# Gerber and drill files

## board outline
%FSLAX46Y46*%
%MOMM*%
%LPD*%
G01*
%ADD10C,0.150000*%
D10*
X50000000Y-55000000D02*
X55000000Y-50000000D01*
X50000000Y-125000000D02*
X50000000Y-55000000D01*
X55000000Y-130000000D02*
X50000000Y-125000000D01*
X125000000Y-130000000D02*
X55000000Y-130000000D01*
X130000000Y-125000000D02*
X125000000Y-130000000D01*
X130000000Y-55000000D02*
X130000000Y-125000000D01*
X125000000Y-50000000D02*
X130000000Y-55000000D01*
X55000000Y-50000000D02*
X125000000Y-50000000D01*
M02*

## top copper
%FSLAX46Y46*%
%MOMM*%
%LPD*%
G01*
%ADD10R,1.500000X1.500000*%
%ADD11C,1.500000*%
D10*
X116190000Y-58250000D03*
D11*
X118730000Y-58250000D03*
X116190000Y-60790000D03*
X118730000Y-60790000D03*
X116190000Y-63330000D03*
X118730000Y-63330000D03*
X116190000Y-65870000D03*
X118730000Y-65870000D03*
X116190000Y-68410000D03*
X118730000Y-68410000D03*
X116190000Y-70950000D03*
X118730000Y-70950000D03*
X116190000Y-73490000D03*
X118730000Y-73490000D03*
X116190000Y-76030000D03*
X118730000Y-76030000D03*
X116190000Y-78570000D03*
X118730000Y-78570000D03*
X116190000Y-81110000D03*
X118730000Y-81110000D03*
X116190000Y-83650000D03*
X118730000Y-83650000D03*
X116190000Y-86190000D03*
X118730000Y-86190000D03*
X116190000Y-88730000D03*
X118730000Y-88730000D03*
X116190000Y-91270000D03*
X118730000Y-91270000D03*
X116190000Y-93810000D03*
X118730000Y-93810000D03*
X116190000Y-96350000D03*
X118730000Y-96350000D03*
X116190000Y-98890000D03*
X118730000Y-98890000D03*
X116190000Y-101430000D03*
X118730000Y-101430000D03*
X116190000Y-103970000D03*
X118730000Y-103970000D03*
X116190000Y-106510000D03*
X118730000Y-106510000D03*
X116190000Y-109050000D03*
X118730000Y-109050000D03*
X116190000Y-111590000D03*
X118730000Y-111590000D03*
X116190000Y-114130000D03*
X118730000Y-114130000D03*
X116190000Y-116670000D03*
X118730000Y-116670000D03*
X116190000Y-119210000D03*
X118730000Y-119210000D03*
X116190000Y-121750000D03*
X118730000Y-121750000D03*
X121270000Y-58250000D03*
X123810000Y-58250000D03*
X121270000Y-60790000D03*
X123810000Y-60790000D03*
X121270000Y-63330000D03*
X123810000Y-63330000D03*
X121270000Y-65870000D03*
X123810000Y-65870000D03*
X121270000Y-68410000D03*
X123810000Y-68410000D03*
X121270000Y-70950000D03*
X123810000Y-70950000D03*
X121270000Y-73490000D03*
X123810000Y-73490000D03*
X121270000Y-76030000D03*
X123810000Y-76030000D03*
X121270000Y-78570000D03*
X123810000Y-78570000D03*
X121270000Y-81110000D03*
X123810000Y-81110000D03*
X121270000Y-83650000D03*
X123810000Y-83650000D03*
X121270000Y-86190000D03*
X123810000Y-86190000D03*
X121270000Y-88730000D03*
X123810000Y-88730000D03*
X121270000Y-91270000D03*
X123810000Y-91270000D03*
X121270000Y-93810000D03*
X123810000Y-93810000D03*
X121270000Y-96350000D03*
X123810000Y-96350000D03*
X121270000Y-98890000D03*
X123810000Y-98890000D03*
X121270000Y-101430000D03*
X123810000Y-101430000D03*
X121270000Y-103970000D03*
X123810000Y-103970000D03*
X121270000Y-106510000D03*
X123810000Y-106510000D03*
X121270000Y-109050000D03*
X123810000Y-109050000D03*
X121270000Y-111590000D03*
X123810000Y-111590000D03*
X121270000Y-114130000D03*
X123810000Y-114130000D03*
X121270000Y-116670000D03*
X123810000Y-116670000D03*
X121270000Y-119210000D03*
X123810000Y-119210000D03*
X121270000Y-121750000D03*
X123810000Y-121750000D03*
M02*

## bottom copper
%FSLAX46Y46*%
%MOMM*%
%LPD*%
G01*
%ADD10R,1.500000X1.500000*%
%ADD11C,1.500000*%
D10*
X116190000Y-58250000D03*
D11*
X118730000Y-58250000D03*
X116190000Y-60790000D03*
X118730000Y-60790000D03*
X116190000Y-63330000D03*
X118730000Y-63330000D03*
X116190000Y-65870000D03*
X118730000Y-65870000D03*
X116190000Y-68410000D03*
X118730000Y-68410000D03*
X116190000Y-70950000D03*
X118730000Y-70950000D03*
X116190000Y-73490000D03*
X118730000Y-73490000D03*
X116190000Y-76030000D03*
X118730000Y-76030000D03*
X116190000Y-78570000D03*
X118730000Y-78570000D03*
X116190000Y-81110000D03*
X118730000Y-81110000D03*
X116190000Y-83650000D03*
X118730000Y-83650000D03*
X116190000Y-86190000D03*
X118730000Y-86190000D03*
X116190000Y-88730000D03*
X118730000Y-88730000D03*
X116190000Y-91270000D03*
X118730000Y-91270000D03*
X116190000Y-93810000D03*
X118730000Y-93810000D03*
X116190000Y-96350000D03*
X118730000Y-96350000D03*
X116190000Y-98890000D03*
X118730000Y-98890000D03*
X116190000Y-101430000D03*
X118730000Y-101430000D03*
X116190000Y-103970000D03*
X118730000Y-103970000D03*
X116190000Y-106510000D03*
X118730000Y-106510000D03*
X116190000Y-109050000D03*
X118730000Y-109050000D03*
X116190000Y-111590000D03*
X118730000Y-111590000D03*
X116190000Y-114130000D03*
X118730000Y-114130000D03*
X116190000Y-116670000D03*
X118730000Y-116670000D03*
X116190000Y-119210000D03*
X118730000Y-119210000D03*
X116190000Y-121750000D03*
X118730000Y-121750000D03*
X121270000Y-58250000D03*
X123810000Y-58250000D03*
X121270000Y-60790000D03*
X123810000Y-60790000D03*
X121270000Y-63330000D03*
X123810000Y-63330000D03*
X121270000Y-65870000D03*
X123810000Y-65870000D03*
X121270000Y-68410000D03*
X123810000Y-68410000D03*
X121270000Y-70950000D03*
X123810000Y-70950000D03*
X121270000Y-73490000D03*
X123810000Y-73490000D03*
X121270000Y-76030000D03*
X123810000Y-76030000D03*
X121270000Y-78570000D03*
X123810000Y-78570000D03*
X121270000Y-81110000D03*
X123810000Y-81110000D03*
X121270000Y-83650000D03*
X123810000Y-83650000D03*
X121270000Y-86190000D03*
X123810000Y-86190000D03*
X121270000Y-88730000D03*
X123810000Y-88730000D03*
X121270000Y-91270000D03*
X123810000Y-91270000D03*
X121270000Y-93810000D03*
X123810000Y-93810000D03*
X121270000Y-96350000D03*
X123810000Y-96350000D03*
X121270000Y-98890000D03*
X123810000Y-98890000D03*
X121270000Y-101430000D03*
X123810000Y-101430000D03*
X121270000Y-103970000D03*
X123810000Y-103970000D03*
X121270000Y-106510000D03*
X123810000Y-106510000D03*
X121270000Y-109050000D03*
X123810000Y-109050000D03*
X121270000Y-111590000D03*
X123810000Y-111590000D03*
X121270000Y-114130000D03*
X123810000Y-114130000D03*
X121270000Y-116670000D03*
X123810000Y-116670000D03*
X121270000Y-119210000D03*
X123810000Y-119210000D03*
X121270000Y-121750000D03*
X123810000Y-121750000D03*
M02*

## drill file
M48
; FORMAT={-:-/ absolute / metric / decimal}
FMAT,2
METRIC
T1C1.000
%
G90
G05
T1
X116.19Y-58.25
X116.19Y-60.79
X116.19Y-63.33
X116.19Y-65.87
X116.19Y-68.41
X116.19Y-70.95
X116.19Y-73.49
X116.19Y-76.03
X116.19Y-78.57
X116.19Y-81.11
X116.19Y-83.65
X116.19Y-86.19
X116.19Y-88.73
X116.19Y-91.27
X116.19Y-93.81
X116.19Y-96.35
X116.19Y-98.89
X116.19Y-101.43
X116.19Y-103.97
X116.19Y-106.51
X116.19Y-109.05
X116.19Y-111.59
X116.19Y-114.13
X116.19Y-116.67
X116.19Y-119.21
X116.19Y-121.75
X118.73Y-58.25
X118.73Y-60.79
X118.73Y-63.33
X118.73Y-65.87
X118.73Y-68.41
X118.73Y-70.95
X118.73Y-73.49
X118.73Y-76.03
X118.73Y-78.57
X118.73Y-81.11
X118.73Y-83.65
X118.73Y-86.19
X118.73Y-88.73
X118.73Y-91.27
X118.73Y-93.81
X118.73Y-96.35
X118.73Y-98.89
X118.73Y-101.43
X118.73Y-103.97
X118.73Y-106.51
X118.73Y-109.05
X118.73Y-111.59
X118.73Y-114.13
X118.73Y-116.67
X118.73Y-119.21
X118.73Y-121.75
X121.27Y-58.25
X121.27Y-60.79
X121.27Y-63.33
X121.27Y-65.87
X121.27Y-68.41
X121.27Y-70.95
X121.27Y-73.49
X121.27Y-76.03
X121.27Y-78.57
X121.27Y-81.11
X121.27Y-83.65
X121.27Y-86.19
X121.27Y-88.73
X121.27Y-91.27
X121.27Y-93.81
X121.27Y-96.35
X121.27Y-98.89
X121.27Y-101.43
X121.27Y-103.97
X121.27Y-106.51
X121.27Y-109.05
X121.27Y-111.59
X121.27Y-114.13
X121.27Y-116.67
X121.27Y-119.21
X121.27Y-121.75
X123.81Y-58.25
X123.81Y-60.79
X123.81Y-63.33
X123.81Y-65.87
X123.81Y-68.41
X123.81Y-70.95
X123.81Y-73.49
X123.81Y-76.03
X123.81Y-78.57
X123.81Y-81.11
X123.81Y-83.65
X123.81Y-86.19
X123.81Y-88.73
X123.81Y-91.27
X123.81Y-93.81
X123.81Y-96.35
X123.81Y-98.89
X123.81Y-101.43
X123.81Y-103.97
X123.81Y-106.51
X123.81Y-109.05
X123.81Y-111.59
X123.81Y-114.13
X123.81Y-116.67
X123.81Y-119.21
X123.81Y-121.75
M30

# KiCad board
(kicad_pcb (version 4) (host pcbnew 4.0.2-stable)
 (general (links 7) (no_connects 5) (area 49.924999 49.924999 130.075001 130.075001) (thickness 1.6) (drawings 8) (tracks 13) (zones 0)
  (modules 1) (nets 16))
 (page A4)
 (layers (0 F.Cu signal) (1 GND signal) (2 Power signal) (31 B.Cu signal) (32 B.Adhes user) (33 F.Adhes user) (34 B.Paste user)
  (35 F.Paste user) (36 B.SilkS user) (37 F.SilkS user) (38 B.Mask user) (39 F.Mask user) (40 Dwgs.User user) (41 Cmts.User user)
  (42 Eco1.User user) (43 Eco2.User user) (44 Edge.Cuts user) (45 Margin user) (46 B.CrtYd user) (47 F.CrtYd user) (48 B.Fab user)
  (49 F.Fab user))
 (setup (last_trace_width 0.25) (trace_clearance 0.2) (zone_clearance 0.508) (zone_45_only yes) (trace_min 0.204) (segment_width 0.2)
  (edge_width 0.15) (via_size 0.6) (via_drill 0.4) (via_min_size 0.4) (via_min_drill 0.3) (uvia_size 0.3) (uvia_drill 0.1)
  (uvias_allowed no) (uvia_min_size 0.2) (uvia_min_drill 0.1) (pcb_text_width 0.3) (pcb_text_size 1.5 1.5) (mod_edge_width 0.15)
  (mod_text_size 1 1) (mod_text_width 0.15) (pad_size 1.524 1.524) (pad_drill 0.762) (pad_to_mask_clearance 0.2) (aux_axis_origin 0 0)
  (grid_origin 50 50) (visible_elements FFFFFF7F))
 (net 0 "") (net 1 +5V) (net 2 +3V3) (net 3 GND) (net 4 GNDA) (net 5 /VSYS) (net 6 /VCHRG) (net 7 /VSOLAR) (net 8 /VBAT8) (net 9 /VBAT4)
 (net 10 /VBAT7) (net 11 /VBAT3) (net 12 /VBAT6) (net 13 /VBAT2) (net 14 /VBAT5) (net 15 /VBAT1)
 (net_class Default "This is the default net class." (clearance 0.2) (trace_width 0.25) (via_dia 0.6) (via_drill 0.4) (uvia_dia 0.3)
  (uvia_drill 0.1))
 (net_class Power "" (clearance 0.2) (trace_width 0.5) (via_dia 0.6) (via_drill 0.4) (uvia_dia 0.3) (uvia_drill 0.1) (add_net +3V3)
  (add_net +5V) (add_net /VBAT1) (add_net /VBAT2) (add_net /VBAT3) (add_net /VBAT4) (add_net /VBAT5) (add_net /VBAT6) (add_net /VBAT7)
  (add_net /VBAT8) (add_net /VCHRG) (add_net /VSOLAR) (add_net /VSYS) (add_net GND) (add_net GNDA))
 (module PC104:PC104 (layer F.Cu) (at 120 90)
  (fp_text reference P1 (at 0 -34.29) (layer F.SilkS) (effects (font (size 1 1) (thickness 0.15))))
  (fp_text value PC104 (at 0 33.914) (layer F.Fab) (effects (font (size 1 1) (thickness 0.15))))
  (pad 1A thru_hole rect (at -3.81 -31.75) (size 1.5 1.5) (drill 1) (layers *.Cu *.Mask F.SilkS))
  (pad 1B thru_hole circle (at -1.27 -31.75) (size 1.5 1.5) (drill 1) (layers *.Cu *.Mask F.SilkS))
  (pad 2A thru_hole circle (at -3.81 -29.21) (size 1.5 1.5) (drill 1) (layers *.Cu *.Mask F.SilkS))
  (pad 2B thru_hole circle (at -1.27 -29.21) (size 1.5 1.5) (drill 1) (layers *.Cu *.Mask F.SilkS))
  (pad 3A thru_hole circle (at -3.81 -26.67) (size 1.5 1.5) (drill 1) (layers *.Cu *.Mask F.SilkS))
  (pad 3B thru_hole circle (at -1.27 -26.67) (size 1.5 1.5) (drill 1) (layers *.Cu *.Mask F.SilkS))
  (pad 4A thru_hole circle (at -3.81 -24.13) (size 1.5 1.5) (drill 1) (layers *.Cu *.Mask F.SilkS))
  (pad 4B thru_hole circle (at -1.27 -24.13) (size 1.5 1.5) (drill 1) (layers *.Cu *.Mask F.SilkS))
  (pad 5A thru_hole circle (at -3.81 -21.59) (size 1.5 1.5) (drill 1) (layers *.Cu *.Mask F.SilkS))
  (pad 5B thru_hole circle (at -1.27 -21.59) (size 1.5 1.5) (drill 1) (layers *.Cu *.Mask F.SilkS))
  (pad 6A thru_hole circle (at -3.81 -19.05) (size 1.5 1.5) (drill 1) (layers *.Cu *.Mask F.SilkS))
  (pad 6B thru_hole circle (at -1.27 -19.05) (size 1.5 1.5) (drill 1) (layers *.Cu *.Mask F.SilkS))
  (pad 7A thru_hole circle (at -3.81 -16.51) (size 1.5 1.5) (drill 1) (layers *.Cu *.Mask F.SilkS))
  (pad 7B thru_hole circle (at -1.27 -16.51) (size 1.5 1.5) (drill 1) (layers *.Cu *.Mask F.SilkS))
  (pad 8A thru_hole circle (at -3.81 -13.97) (size 1.5 1.5) (drill 1) (layers *.Cu *.Mask F.SilkS))
  (pad 8B thru_hole circle (at -1.27 -13.97) (size 1.5 1.5) (drill 1) (layers *.Cu *.Mask F.SilkS))
  (pad 9A thru_hole circle (at -3.81 -11.43) (size 1.5 1.5) (drill 1) (layers *.Cu *.Mask F.SilkS))
  (pad 9B thru_hole circle (at -1.27 -11.43) (size 1.5 1.5) (drill 1) (layers *.Cu *.Mask F.SilkS))
  (pad 10A thru_hole circle (at -3.81 -8.89) (size 1.5 1.5) (drill 1) (layers *.Cu *.Mask F.SilkS))
  (pad 10B thru_hole circle (at -1.27 -8.89) (size 1.5 1.5) (drill 1) (layers *.Cu *.Mask F.SilkS))
  (pad 11A thru_hole circle (at -3.81 -6.35) (size 1.5 1.5) (drill 1) (layers *.Cu *.Mask F.SilkS))
  (pad 11B thru_hole circle (at -1.27 -6.35) (size 1.5 1.5) (drill 1) (layers *.Cu *.Mask F.SilkS))
  (pad 12A thru_hole circle (at -3.81 -3.81) (size 1.5 1.5) (drill 1) (layers *.Cu *.Mask F.SilkS))
  (pad 12B thru_hole circle (at -1.27 -3.81) (size 1.5 1.5) (drill 1) (layers *.Cu *.Mask F.SilkS))
  (pad 13A thru_hole circle (at -3.81 -1.27) (size 1.5 1.5) (drill 1) (layers *.Cu *.Mask F.SilkS))
  (pad 13B thru_hole circle (at -1.27 -1.27) (size 1.5 1.5) (drill 1) (layers *.Cu *.Mask F.SilkS))
  (pad 14A thru_hole circle (at -3.81 1.27) (size 1.5 1.5) (drill 1) (layers *.Cu *.Mask F.SilkS))
  (pad 14B thru_hole circle (at -1.27 1.27) (size 1.5 1.5) (drill 1) (layers *.Cu *.Mask F.SilkS))
  (pad 15A thru_hole circle (at -3.81 3.81) (size 1.5 1.5) (drill 1) (layers *.Cu *.Mask F.SilkS))
  (pad 15B thru_hole circle (at -1.27 3.81) (size 1.5 1.5) (drill 1) (layers *.Cu *.Mask F.SilkS))
  (pad 16A thru_hole circle (at -3.81 6.35) (size 1.5 1.5) (drill 1) (layers *.Cu *.Mask F.SilkS))
  (pad 16B thru_hole circle (at -1.27 6.35) (size 1.5 1.5) (drill 1) (layers *.Cu *.Mask F.SilkS))
  (pad 17A thru_hole circle (at -3.81 8.89) (size 1.5 1.5) (drill 1) (layers *.Cu *.Mask F.SilkS))
  (pad 17B thru_hole circle (at -1.27 8.89) (size 1.5 1.5) (drill 1) (layers *.Cu *.Mask F.SilkS))
  (pad 18A thru_hole circle (at -3.81 11.43) (size 1.5 1.5) (drill 1) (layers *.Cu *.Mask F.SilkS))
  (pad 18B thru_hole circle (at -1.27 11.43) (size 1.5 1.5) (drill 1) (layers *.Cu *.Mask F.SilkS))
  (pad 19A thru_hole circle (at -3.81 13.97) (size 1.5 1.5) (drill 1) (layers *.Cu *.Mask F.SilkS))
  (pad 19B thru_hole circle (at -1.27 13.97) (size 1.5 1.5) (drill 1) (layers *.Cu *.Mask F.SilkS))
  (pad 20A thru_hole circle (at -3.81 16.51) (size 1.5 1.5) (drill 1) (layers *.Cu *.Mask F.SilkS))
  (pad 20B thru_hole circle (at -1.27 16.51) (size 1.5 1.5) (drill 1) (layers *.Cu *.Mask F.SilkS))
  (pad 21A thru_hole circle (at -3.81 19.05) (size 1.5 1.5) (drill 1) (layers *.Cu *.Mask F.SilkS))
  (pad 21B thru_hole circle (at -1.27 19.05) (size 1.5 1.5) (drill 1) (layers *.Cu *.Mask F.SilkS))
  (pad 22A thru_hole circle (at -3.81 21.59) (size 1.5 1.5) (drill 1) (layers *.Cu *.Mask F.SilkS))
  (pad 22B thru_hole circle (at -1.27 21.59) (size 1.5 1.5) (drill 1) (layers *.Cu *.Mask F.SilkS))
  (pad 23A thru_hole circle (at -3.81 24.13) (size 1.5 1.5) (drill 1) (layers *.Cu *.Mask F.SilkS))
  (pad 23B thru_hole circle (at -1.27 24.13) (size 1.5 1.5) (drill 1) (layers *.Cu *.Mask F.SilkS))
  (pad 24A thru_hole circle (at -3.81 26.67) (size 1.5 1.5) (drill 1) (layers *.Cu *.Mask F.SilkS))
  (pad 24B thru_hole circle (at -1.27 26.67) (size 1.5 1.5) (drill 1) (layers *.Cu *.Mask F.SilkS))
  (pad 25A thru_hole circle (at -3.81 29.21) (size 1.5 1.5) (drill 1) (layers *.Cu *.Mask F.SilkS))
  (pad 25B thru_hole circle (at -1.27 29.21) (size 1.5 1.5) (drill 1) (layers *.Cu *.Mask F.SilkS))
  (pad 26A thru_hole circle (at -3.81 31.75) (size 1.5 1.5) (drill 1) (layers *.Cu *.Mask F.SilkS))
  (pad 26B thru_hole circle (at -1.27 31.75) (size 1.5 1.5) (drill 1) (layers *.Cu *.Mask F.SilkS))
  (pad 1C thru_hole circle (at 1.27 -31.75) (size 1.5 1.5) (drill 1) (layers *.Cu *.Mask F.SilkS))
  (pad 1D thru_hole circle (at 3.81 -31.75) (size 1.5 1.5) (drill 1) (layers *.Cu *.Mask F.SilkS))
  (pad 2C thru_hole circle (at 1.27 -29.21) (size 1.5 1.5) (drill 1) (layers *.Cu *.Mask F.SilkS))
  (pad 2D thru_hole circle (at 3.81 -29.21) (size 1.5 1.5) (drill 1) (layers *.Cu *.Mask F.SilkS))
  (pad 3C thru_hole circle (at 1.27 -26.67) (size 1.5 1.5) (drill 1) (layers *.Cu *.Mask F.SilkS))
  (pad 3D thru_hole circle (at 3.81 -26.67) (size 1.5 1.5) (drill 1) (layers *.Cu *.Mask F.SilkS))
  (pad 4C thru_hole circle (at 1.27 -24.13) (size 1.5 1.5) (drill 1) (layers *.Cu *.Mask F.SilkS))
  (pad 4D thru_hole circle (at 3.81 -24.13) (size 1.5 1.5) (drill 1) (layers *.Cu *.Mask F.SilkS))
  (pad 5C thru_hole circle (at 1.27 -21.59) (size 1.5 1.5) (drill 1) (layers *.Cu *.Mask F.SilkS))
  (pad 5D thru_hole circle (at 3.81 -21.59) (size 1.5 1.5) (drill 1) (layers *.Cu *.Mask F.SilkS))
  (pad 6C thru_hole circle (at 1.27 -19.05) (size 1.5 1.5) (drill 1) (layers *.Cu *.Mask F.SilkS))
  (pad 6D thru_hole circle (at 3.81 -19.05) (size 1.5 1.5) (drill 1) (layers *.Cu *.Mask F.SilkS))
  (pad 7C thru_hole circle (at 1.27 -16.51) (size 1.5 1.5) (drill 1) (layers *.Cu *.Mask F.SilkS))
  (pad 7D thru_hole circle (at 3.81 -16.51) (size 1.5 1.5) (drill 1) (layers *.Cu *.Mask F.SilkS))
  (pad 8C thru_hole circle (at 1.27 -13.97) (size 1.5 1.5) (drill 1) (layers *.Cu *.Mask F.SilkS))
  (pad 8D thru_hole circle (at 3.81 -13.97) (size 1.5 1.5) (drill 1) (layers *.Cu *.Mask F.SilkS))
  (pad 9C thru_hole circle (at 1.27 -11.43) (size 1.5 1.5) (drill 1) (layers *.Cu *.Mask F.SilkS))
  (pad 9D thru_hole circle (at 3.81 -11.43) (size 1.5 1.5) (drill 1) (layers *.Cu *.Mask F.SilkS))
  (pad 10C thru_hole circle (at 1.27 -8.89) (size 1.5 1.5) (drill 1) (layers *.Cu *.Mask F.SilkS))
  (pad 10D thru_hole circle (at 3.81 -8.89) (size 1.5 1.5) (drill 1) (layers *.Cu *.Mask F.SilkS))
  (pad 11C thru_hole circle (at 1.27 -6.35) (size 1.5 1.5) (drill 1) (layers *.Cu *.Mask F.SilkS))
  (pad 11D thru_hole circle (at 3.81 -6.35) (size 1.5 1.5) (drill 1) (layers *.Cu *.Mask F.SilkS))
  (pad 12C thru_hole circle (at 1.27 -3.81) (size 1.5 1.5) (drill 1) (layers *.Cu *.Mask F.SilkS))
  (pad 12D thru_hole circle (at 3.81 -3.81) (size 1.5 1.5) (drill 1) (layers *.Cu *.Mask F.SilkS))
  (pad 13C thru_hole circle (at 1.27 -1.27) (size 1.5 1.5) (drill 1) (layers *.Cu *.Mask F.SilkS) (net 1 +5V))
  (pad 13D thru_hole circle (at 3.81 -1.27) (size 1.5 1.5) (drill 1) (layers *.Cu *.Mask F.SilkS) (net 1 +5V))
  (pad 14C thru_hole circle (at 1.27 1.27) (size 1.5 1.5) (drill 1) (layers *.Cu *.Mask F.SilkS) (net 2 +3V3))
  (pad 14D thru_hole circle (at 3.81 1.27) (size 1.5 1.5) (drill 1) (layers *.Cu *.Mask F.SilkS) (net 2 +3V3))
  (pad 15C thru_hole circle (at 1.27 3.81) (size 1.5 1.5) (drill 1) (layers *.Cu *.Mask F.SilkS) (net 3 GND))
  (pad 15D thru_hole circle (at 3.81 3.81) (size 1.5 1.5) (drill 1) (layers *.Cu *.Mask F.SilkS) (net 3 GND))
  (pad 16C thru_hole circle (at 1.27 6.35) (size 1.5 1.5) (drill 1) (layers *.Cu *.Mask F.SilkS) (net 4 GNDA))
  (pad 16D thru_hole circle (at 3.81 6.35) (size 1.5 1.5) (drill 1) (layers *.Cu *.Mask F.SilkS) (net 3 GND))
  (pad 17C thru_hole circle (at 1.27 8.89) (size 1.5 1.5) (drill 1) (layers *.Cu *.Mask F.SilkS) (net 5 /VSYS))
  (pad 17D thru_hole circle (at 3.81 8.89) (size 1.5 1.5) (drill 1) (layers *.Cu *.Mask F.SilkS) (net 5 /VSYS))
  (pad 18C thru_hole circle (at 1.27 11.43) (size 1.5 1.5) (drill 1) (layers *.Cu *.Mask F.SilkS) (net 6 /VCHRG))
  (pad 18D thru_hole circle (at 3.81 11.43) (size 1.5 1.5) (drill 1) (layers *.Cu *.Mask F.SilkS) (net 6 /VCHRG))
  (pad 19C thru_hole circle (at 1.27 13.97) (size 1.5 1.5) (drill 1) (layers *.Cu *.Mask F.SilkS) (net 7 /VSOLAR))
  (pad 19D thru_hole circle (at 3.81 13.97) (size 1.5 1.5) (drill 1) (layers *.Cu *.Mask F.SilkS) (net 7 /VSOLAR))
  (pad 20C thru_hole circle (at 1.27 16.51) (size 1.5 1.5) (drill 1) (layers *.Cu *.Mask F.SilkS) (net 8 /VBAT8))
  (pad 20D thru_hole circle (at 3.81 16.51) (size 1.5 1.5) (drill 1) (layers *.Cu *.Mask F.SilkS) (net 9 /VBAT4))
  (pad 21C thru_hole circle (at 1.27 19.05) (size 1.5 1.5) (drill 1) (layers *.Cu *.Mask F.SilkS) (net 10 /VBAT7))
  (pad 21D thru_hole circle (at 3.81 19.05) (size 1.5 1.5) (drill 1) (layers *.Cu *.Mask F.SilkS) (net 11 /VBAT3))
  (pad 22C thru_hole circle (at 1.27 21.59) (size 1.5 1.5) (drill 1) (layers *.Cu *.Mask F.SilkS) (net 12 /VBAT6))
  (pad 22D thru_hole circle (at 3.81 21.59) (size 1.5 1.5) (drill 1) (layers *.Cu *.Mask F.SilkS) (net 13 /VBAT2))
  (pad 23C thru_hole circle (at 1.27 24.13) (size 1.5 1.5) (drill 1) (layers *.Cu *.Mask F.SilkS) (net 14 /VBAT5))
  (pad 23D thru_hole circle (at 3.81 24.13) (size 1.5 1.5) (drill 1) (layers *.Cu *.Mask F.SilkS) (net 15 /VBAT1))
  (pad 24C thru_hole circle (at 1.27 26.67) (size 1.5 1.5) (drill 1) (layers *.Cu *.Mask F.SilkS))
  (pad 24D thru_hole circle (at 3.81 26.67) (size 1.5 1.5) (drill 1) (layers *.Cu *.Mask F.SilkS))
  (pad 25C thru_hole circle (at 1.27 29.21) (size 1.5 1.5) (drill 1) (layers *.Cu *.Mask F.SilkS))
  (pad 25D thru_hole circle (at 3.81 29.21) (size 1.5 1.5) (drill 1) (layers *.Cu *.Mask F.SilkS))
  (pad 26C thru_hole circle (at 1.27 31.75) (size 1.5 1.5) (drill 1) (layers *.Cu *.Mask F.SilkS))
  (pad 26D thru_hole circle (at 3.81 31.75) (size 1.5 1.5) (drill 1) (layers *.Cu *.Mask F.SilkS)))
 (gr_line (start 50 55) (end 55 50) (layer Edge.Cuts) (width 0.15))
 (gr_line (start 50 125) (end 50 55) (layer Edge.Cuts) (width 0.15))
 (gr_line (start 55 130) (end 50 125) (layer Edge.Cuts) (width 0.15))
 (gr_line (start 125 130) (end 55 130) (layer Edge.Cuts) (width 0.15))
 (gr_line (start 130 125) (end 125 130) (layer Edge.Cuts) (width 0.15))
 (gr_line (start 130 55) (end 130 125) (layer Edge.Cuts) (width 0.15))
 (gr_line (start 125 50) (end 130 55) (layer Edge.Cuts) (width 0.15))
 (gr_line (start 55 50) (end 125 50) (layer Edge.Cuts) (width 0.15))
 (segment (start 123.81 88.73) (end 121.27 88.73) (width 0.5) (layer Power) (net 1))
 (segment (start 123.81 91.27) (end 121.27 91.27) (width 0.5) (layer Power) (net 2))
 (segment (start 120.069999 95.010001) (end 120.144998 95.085) (width 0.5) (layer GND) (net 3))
 (segment (start 120.069999 95.010001) (end 119.995 95.085) (width 0.5) (layer GND) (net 3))
 (segment (start 119.995 95.085) (end 114.135 95.085) (width 0.5) (layer GND) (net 3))
 (segment (start 120.005 92.545) (end 114.135 92.545) (width 0.5) (layer GND) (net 3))
 (segment (start 121.27 93.81) (end 120.005 92.545) (width 0.5) (layer GND) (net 3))
 (segment (start 121.27 93.81) (end 120.069999 95.010001) (width 0.5) (layer GND) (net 3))
 (segment (start 123.81 98.89) (end 121.27 98.89) (width 0.5) (layer Power) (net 5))
 (segment (start 123.81 101.43) (end 121.27 101.43) (width 0.5) (layer Power) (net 6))
 (segment (start 123.81 103.97) (end 121.27 103.97) (width 0.5) (layer Power) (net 7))
 (segment (start 121.27 96.35) (end 119.995 97.625) (width 0.5) (layer GND) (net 4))
 (segment (start 119.995 97.625) (end 114.135 97.625) (width 0.5) (layer GND) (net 4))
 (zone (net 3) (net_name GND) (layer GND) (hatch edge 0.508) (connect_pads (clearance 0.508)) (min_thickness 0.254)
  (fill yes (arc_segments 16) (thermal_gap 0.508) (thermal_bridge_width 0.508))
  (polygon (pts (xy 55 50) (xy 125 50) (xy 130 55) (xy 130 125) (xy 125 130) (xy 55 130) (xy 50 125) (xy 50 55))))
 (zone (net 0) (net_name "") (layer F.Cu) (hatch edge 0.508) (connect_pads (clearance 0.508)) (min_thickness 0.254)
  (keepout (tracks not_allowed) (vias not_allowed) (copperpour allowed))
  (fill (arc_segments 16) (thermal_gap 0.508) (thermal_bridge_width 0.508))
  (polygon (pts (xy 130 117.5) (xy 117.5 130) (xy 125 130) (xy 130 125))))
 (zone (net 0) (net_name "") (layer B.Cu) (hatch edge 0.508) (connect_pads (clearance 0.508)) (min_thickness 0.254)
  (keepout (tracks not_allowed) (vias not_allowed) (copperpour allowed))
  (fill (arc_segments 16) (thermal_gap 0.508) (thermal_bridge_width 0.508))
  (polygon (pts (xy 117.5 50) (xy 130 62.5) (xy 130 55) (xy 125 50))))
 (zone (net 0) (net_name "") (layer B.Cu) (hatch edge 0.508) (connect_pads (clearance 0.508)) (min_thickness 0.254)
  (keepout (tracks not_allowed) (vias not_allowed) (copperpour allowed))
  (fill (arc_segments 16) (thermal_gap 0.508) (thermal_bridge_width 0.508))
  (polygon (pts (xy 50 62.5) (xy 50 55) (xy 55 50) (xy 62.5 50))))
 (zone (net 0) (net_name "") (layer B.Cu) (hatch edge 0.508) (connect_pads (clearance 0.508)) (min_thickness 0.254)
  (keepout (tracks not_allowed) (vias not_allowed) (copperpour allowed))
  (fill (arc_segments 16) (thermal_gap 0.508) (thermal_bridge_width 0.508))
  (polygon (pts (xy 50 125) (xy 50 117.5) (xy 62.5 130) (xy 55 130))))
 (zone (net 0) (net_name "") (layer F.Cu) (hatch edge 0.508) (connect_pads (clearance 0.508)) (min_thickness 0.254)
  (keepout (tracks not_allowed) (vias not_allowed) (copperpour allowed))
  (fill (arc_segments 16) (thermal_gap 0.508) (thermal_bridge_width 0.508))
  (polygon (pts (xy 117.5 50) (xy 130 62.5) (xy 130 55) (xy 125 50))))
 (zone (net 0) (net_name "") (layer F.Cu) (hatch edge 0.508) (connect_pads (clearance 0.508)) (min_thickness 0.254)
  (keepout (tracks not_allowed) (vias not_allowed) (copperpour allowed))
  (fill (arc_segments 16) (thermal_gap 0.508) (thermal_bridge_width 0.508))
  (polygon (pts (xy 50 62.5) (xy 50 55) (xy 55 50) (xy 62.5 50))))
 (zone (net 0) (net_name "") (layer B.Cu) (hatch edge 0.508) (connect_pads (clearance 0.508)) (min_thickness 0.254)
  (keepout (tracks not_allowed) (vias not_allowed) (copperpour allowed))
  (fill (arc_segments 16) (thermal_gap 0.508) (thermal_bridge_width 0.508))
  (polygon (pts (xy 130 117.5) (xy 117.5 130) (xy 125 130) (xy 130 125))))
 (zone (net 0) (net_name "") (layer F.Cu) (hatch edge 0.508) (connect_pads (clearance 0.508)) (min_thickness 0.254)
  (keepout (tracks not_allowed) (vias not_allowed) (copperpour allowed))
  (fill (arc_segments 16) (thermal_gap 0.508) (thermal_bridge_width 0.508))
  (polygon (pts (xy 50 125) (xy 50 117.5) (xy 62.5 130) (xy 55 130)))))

